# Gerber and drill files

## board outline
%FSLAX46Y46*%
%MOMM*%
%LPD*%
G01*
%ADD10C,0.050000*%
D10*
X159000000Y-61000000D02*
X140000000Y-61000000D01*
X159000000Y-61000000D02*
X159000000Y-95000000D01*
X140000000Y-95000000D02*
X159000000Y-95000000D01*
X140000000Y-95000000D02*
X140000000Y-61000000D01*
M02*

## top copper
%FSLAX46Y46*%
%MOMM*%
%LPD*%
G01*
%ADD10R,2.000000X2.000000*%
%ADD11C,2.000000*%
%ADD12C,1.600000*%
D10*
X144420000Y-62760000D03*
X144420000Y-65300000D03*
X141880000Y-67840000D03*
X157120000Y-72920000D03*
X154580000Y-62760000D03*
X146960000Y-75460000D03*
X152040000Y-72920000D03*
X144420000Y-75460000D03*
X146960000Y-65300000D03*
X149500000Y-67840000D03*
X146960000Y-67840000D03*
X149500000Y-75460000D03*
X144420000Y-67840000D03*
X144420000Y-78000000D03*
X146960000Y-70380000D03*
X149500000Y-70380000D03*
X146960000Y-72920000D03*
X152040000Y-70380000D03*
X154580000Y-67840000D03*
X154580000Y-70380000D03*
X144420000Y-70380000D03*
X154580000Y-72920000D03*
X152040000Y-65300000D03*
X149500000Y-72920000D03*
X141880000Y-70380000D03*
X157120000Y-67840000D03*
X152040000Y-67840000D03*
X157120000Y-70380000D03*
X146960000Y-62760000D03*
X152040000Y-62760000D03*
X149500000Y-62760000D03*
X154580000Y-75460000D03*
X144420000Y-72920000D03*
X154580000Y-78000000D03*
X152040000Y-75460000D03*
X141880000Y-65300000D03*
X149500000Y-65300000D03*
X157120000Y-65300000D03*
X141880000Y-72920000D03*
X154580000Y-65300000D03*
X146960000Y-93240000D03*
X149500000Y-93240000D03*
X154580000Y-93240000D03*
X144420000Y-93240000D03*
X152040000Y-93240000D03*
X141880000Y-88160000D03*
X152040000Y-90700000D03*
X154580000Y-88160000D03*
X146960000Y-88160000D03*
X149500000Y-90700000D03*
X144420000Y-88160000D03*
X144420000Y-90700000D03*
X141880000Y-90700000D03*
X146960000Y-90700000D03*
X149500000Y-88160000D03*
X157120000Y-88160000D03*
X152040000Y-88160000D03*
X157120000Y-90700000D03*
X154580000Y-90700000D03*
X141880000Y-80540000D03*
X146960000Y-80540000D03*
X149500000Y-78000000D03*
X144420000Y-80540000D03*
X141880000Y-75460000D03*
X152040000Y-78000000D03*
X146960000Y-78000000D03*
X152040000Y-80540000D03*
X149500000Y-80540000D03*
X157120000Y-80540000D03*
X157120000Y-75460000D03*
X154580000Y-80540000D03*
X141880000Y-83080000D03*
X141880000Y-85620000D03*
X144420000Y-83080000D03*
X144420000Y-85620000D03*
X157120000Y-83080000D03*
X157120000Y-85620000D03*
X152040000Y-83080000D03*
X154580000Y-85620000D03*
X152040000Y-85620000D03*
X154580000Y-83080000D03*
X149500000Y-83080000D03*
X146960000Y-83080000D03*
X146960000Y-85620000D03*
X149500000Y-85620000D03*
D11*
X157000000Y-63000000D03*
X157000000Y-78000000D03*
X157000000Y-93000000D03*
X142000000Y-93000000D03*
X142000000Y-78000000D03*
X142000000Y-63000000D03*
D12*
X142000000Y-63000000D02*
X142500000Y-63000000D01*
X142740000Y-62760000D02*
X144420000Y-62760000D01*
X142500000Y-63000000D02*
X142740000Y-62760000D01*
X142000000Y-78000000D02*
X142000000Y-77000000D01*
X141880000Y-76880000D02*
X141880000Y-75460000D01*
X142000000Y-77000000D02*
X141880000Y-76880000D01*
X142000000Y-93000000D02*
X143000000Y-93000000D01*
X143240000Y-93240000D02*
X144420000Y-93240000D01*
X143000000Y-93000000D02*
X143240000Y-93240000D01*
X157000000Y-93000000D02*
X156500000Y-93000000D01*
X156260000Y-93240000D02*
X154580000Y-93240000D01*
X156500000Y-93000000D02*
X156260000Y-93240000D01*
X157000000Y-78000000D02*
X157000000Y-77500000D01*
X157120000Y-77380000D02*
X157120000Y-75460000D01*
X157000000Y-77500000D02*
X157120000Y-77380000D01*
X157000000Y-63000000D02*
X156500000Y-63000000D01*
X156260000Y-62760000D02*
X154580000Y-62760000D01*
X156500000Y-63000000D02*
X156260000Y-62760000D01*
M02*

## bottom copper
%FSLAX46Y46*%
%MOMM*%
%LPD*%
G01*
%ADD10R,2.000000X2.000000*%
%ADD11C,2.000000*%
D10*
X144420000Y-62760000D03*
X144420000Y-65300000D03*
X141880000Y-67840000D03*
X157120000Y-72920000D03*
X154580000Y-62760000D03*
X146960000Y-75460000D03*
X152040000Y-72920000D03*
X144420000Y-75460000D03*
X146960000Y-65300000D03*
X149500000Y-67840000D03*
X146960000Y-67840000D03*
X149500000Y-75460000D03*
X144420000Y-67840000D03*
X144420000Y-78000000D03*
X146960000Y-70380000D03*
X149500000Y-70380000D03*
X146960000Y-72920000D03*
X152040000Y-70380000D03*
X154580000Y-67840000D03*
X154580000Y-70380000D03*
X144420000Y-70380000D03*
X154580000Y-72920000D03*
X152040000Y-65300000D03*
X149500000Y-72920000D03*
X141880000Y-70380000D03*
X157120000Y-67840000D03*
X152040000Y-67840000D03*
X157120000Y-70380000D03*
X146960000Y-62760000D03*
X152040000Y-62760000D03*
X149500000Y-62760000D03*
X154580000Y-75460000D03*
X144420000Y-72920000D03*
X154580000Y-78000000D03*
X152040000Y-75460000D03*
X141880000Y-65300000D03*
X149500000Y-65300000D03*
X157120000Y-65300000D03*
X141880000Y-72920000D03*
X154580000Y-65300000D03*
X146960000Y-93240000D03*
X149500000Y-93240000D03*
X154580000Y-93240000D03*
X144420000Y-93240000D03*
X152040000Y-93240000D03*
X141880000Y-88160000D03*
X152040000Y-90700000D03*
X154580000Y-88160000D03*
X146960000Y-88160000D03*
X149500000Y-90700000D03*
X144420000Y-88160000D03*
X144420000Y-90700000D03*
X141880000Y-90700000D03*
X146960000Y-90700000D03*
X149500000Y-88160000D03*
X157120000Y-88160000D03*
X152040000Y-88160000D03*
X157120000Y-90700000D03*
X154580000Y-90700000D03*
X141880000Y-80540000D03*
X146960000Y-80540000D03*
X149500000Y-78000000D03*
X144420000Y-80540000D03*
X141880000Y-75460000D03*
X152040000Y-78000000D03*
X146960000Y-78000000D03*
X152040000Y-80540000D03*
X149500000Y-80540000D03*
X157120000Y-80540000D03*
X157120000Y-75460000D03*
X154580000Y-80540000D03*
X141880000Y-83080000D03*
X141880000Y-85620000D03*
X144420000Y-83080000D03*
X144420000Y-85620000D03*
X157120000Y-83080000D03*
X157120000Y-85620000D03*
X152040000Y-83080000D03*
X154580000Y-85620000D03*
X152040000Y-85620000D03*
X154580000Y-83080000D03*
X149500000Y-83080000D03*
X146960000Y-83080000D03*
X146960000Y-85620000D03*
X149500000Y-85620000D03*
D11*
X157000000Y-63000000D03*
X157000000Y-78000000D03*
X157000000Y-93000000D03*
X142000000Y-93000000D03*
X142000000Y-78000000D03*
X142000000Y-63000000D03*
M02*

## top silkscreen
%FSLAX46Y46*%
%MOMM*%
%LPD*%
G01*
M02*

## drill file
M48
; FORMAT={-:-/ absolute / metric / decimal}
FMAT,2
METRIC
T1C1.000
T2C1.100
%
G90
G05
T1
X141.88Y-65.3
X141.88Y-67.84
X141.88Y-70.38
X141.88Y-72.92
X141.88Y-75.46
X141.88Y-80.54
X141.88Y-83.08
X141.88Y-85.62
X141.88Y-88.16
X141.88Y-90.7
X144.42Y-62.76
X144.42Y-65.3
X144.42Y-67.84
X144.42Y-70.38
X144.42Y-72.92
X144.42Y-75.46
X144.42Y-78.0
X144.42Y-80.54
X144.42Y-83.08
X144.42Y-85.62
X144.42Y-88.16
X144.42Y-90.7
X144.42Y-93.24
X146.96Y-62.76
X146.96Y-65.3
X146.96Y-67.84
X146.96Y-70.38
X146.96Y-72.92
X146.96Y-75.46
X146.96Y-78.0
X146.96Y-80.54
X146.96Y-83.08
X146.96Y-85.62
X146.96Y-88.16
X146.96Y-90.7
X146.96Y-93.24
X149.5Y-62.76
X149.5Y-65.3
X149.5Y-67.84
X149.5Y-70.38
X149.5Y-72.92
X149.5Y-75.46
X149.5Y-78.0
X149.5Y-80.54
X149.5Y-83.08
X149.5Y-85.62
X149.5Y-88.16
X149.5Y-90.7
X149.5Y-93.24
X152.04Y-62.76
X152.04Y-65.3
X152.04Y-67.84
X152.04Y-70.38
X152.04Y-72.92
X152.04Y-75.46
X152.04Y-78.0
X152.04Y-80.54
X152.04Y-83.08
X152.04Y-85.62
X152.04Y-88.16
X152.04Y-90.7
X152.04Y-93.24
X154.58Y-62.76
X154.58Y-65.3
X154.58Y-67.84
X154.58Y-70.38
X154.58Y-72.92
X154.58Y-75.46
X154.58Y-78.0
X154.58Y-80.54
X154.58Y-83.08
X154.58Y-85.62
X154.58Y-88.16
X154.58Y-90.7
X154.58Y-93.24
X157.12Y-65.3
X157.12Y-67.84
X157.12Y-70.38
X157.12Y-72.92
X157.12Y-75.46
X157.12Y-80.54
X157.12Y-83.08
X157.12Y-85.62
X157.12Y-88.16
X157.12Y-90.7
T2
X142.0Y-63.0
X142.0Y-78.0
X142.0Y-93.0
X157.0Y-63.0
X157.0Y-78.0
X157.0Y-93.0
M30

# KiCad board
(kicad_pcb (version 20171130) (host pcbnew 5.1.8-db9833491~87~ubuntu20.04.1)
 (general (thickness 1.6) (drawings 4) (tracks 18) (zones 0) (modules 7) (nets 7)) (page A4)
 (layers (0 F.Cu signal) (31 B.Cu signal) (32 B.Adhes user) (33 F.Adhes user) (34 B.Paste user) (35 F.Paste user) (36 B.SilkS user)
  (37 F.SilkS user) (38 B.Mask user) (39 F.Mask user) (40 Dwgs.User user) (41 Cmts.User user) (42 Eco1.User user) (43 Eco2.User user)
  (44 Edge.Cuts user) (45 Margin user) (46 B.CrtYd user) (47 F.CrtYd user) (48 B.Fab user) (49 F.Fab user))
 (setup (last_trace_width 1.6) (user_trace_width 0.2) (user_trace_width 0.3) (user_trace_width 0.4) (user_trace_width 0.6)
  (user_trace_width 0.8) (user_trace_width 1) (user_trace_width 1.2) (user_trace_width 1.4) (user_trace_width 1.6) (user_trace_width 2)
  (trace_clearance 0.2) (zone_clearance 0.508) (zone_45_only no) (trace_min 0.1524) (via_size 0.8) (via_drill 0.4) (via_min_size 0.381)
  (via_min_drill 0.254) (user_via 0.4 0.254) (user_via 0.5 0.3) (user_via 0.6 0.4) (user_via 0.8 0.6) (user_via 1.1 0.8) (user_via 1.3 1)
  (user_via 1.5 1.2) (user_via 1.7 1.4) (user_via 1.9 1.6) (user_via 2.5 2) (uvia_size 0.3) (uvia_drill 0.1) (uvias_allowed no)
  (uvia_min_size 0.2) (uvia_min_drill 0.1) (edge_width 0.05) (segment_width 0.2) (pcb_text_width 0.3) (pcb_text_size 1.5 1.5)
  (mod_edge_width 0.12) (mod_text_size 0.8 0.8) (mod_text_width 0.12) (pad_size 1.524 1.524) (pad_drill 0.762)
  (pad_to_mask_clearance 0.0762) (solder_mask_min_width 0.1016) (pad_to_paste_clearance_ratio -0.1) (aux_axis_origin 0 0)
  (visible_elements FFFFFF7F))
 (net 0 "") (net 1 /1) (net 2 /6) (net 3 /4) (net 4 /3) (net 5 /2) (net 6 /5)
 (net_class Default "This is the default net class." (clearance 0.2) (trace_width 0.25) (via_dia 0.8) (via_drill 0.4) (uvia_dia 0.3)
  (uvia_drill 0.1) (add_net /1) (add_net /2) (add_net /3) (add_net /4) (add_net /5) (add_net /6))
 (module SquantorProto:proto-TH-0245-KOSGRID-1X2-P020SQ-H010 (layer F.Cu) (at 149.5 78)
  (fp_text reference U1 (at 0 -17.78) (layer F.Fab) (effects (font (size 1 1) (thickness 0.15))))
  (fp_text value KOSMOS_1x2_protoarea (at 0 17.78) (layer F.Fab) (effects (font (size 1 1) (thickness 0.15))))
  (pad 1 thru_hole rect (at -5.08 -15.24) (size 2 2) (drill 1) (layers *.Cu *.Mask) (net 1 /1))
  (pad NC thru_hole rect (at -5.08 -12.7) (size 2 2) (drill 1) (layers *.Cu *.Mask))
  (pad NC thru_hole rect (at -7.62 -10.16) (size 2 2) (drill 1) (layers *.Cu *.Mask))
  (pad NC thru_hole rect (at 7.62 -5.08) (size 2 2) (drill 1) (layers *.Cu *.Mask))
  (pad 6 thru_hole rect (at 5.08 -15.24) (size 2 2) (drill 1) (layers *.Cu *.Mask) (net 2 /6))
  (pad NC thru_hole rect (at -2.54 -2.54) (size 2 2) (drill 1) (layers *.Cu *.Mask))
  (pad NC thru_hole rect (at 2.54 -5.08) (size 2 2) (drill 1) (layers *.Cu *.Mask))
  (pad NC thru_hole rect (at -5.08 -2.54) (size 2 2) (drill 1) (layers *.Cu *.Mask))
  (pad NC thru_hole rect (at -2.54 -12.7) (size 2 2) (drill 1) (layers *.Cu *.Mask))
  (pad NC thru_hole rect (at 0 -10.16) (size 2 2) (drill 1) (layers *.Cu *.Mask))
  (pad NC thru_hole rect (at -2.54 -10.16) (size 2 2) (drill 1) (layers *.Cu *.Mask))
  (pad NC thru_hole rect (at 0 -2.54) (size 2 2) (drill 1) (layers *.Cu *.Mask))
  (pad NC thru_hole rect (at -5.08 -10.16) (size 2 2) (drill 1) (layers *.Cu *.Mask))
  (pad NC thru_hole rect (at -5.08 0) (size 2 2) (drill 1) (layers *.Cu *.Mask))
  (pad NC thru_hole rect (at -2.54 -7.62) (size 2 2) (drill 1) (layers *.Cu *.Mask))
  (pad NC thru_hole rect (at 0 -7.62) (size 2 2) (drill 1) (layers *.Cu *.Mask))
  (pad NC thru_hole rect (at -2.54 -5.08) (size 2 2) (drill 1) (layers *.Cu *.Mask))
  (pad NC thru_hole rect (at 2.54 -7.62) (size 2 2) (drill 1) (layers *.Cu *.Mask))
  (pad NC thru_hole rect (at 5.08 -10.16) (size 2 2) (drill 1) (layers *.Cu *.Mask))
  (pad NC thru_hole rect (at 5.08 -7.62) (size 2 2) (drill 1) (layers *.Cu *.Mask))
  (pad NC thru_hole rect (at -5.08 -7.62) (size 2 2) (drill 1) (layers *.Cu *.Mask))
  (pad NC thru_hole rect (at 5.08 -5.08) (size 2 2) (drill 1) (layers *.Cu *.Mask))
  (pad NC thru_hole rect (at 2.54 -12.7) (size 2 2) (drill 1) (layers *.Cu *.Mask))
  (pad NC thru_hole rect (at 0 -5.08) (size 2 2) (drill 1) (layers *.Cu *.Mask))
  (pad NC thru_hole rect (at -7.62 -7.62) (size 2 2) (drill 1) (layers *.Cu *.Mask))
  (pad NC thru_hole rect (at 7.62 -10.16) (size 2 2) (drill 1) (layers *.Cu *.Mask))
  (pad NC thru_hole rect (at 2.54 -10.16) (size 2 2) (drill 1) (layers *.Cu *.Mask))
  (pad NC thru_hole rect (at 7.62 -7.62) (size 2 2) (drill 1) (layers *.Cu *.Mask))
  (pad NC thru_hole rect (at -2.54 -15.24) (size 2 2) (drill 1) (layers *.Cu *.Mask))
  (pad NC thru_hole rect (at 2.54 -15.24) (size 2 2) (drill 1) (layers *.Cu *.Mask))
  (pad NC thru_hole rect (at 0 -15.24) (size 2 2) (drill 1) (layers *.Cu *.Mask))
  (pad NC thru_hole rect (at 5.08 -2.54) (size 2 2) (drill 1) (layers *.Cu *.Mask))
  (pad NC thru_hole rect (at -5.08 -5.08) (size 2 2) (drill 1) (layers *.Cu *.Mask))
  (pad NC thru_hole rect (at 5.08 0) (size 2 2) (drill 1) (layers *.Cu *.Mask))
  (pad NC thru_hole rect (at 2.54 -2.54) (size 2 2) (drill 1) (layers *.Cu *.Mask))
  (pad NC thru_hole rect (at -7.62 -12.7) (size 2 2) (drill 1) (layers *.Cu *.Mask))
  (pad NC thru_hole rect (at 0 -12.7) (size 2 2) (drill 1) (layers *.Cu *.Mask))
  (pad NC thru_hole rect (at 7.62 -12.7) (size 2 2) (drill 1) (layers *.Cu *.Mask))
  (pad NC thru_hole rect (at -7.62 -5.08) (size 2 2) (drill 1) (layers *.Cu *.Mask))
  (pad NC thru_hole rect (at 5.08 -12.7) (size 2 2) (drill 1) (layers *.Cu *.Mask))
  (pad NC thru_hole rect (at -2.54 15.24) (size 2 2) (drill 1) (layers *.Cu *.Mask))
  (pad NC thru_hole rect (at 0 15.24) (size 2 2) (drill 1) (layers *.Cu *.Mask))
  (pad 4 thru_hole rect (at 5.08 15.24) (size 2 2) (drill 1) (layers *.Cu *.Mask) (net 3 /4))
  (pad 3 thru_hole rect (at -5.08 15.24) (size 2 2) (drill 1) (layers *.Cu *.Mask) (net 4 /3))
  (pad NC thru_hole rect (at 2.54 15.24) (size 2 2) (drill 1) (layers *.Cu *.Mask))
  (pad NC thru_hole rect (at -7.62 10.16) (size 2 2) (drill 1) (layers *.Cu *.Mask))
  (pad NC thru_hole rect (at 2.54 12.7) (size 2 2) (drill 1) (layers *.Cu *.Mask))
  (pad NC thru_hole rect (at 5.08 10.16) (size 2 2) (drill 1) (layers *.Cu *.Mask))
  (pad NC thru_hole rect (at -2.54 10.16) (size 2 2) (drill 1) (layers *.Cu *.Mask))
  (pad NC thru_hole rect (at 0 12.7) (size 2 2) (drill 1) (layers *.Cu *.Mask))
  (pad NC thru_hole rect (at -5.08 10.16) (size 2 2) (drill 1) (layers *.Cu *.Mask))
  (pad NC thru_hole rect (at -5.08 12.7) (size 2 2) (drill 1) (layers *.Cu *.Mask))
  (pad NC thru_hole rect (at -7.62 12.7) (size 2 2) (drill 1) (layers *.Cu *.Mask))
  (pad NC thru_hole rect (at -2.54 12.7) (size 2 2) (drill 1) (layers *.Cu *.Mask))
  (pad NC thru_hole rect (at 0 10.16) (size 2 2) (drill 1) (layers *.Cu *.Mask))
  (pad NC thru_hole rect (at 7.62 10.16) (size 2 2) (drill 1) (layers *.Cu *.Mask))
  (pad NC thru_hole rect (at 2.54 10.16) (size 2 2) (drill 1) (layers *.Cu *.Mask))
  (pad NC thru_hole rect (at 7.62 12.7) (size 2 2) (drill 1) (layers *.Cu *.Mask))
  (pad NC thru_hole rect (at 5.08 12.7) (size 2 2) (drill 1) (layers *.Cu *.Mask))
  (pad NC thru_hole rect (at -7.62 2.54) (size 2 2) (drill 1) (layers *.Cu *.Mask))
  (pad NC thru_hole rect (at -2.54 2.54) (size 2 2) (drill 1) (layers *.Cu *.Mask))
  (pad NC thru_hole rect (at 0 0) (size 2 2) (drill 1) (layers *.Cu *.Mask))
  (pad NC thru_hole rect (at -5.08 2.54) (size 2 2) (drill 1) (layers *.Cu *.Mask))
  (pad 2 thru_hole rect (at -7.62 -2.54) (size 2 2) (drill 1) (layers *.Cu *.Mask) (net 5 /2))
  (pad NC thru_hole rect (at 2.54 0) (size 2 2) (drill 1) (layers *.Cu *.Mask))
  (pad NC thru_hole rect (at -2.54 0) (size 2 2) (drill 1) (layers *.Cu *.Mask))
  (pad NC thru_hole rect (at 2.54 2.54) (size 2 2) (drill 1) (layers *.Cu *.Mask))
  (pad NC thru_hole rect (at 0 2.54) (size 2 2) (drill 1) (layers *.Cu *.Mask))
  (pad NC thru_hole rect (at 7.62 2.54) (size 2 2) (drill 1) (layers *.Cu *.Mask))
  (pad 5 thru_hole rect (at 7.62 -2.54) (size 2 2) (drill 1) (layers *.Cu *.Mask) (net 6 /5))
  (pad NC thru_hole rect (at 5.08 2.54) (size 2 2) (drill 1) (layers *.Cu *.Mask))
  (pad NC thru_hole rect (at -7.62 5.08) (size 2 2) (drill 1) (layers *.Cu *.Mask))
  (pad NC thru_hole rect (at -7.62 7.62) (size 2 2) (drill 1) (layers *.Cu *.Mask))
  (pad NC thru_hole rect (at -5.08 5.08) (size 2 2) (drill 1) (layers *.Cu *.Mask))
  (pad NC thru_hole rect (at -5.08 7.62) (size 2 2) (drill 1) (layers *.Cu *.Mask))
  (pad NC thru_hole rect (at 7.62 5.08) (size 2 2) (drill 1) (layers *.Cu *.Mask))
  (pad NC thru_hole rect (at 7.62 7.62) (size 2 2) (drill 1) (layers *.Cu *.Mask))
  (pad NC thru_hole rect (at 2.54 5.08) (size 2 2) (drill 1) (layers *.Cu *.Mask))
  (pad NC thru_hole rect (at 5.08 7.62) (size 2 2) (drill 1) (layers *.Cu *.Mask))
  (pad NC thru_hole rect (at 2.54 7.62) (size 2 2) (drill 1) (layers *.Cu *.Mask))
  (pad NC thru_hole rect (at 5.08 5.08) (size 2 2) (drill 1) (layers *.Cu *.Mask))
  (pad NC thru_hole rect (at 0 5.08) (size 2 2) (drill 1) (layers *.Cu *.Mask))
  (pad NC thru_hole rect (at -2.54 5.08) (size 2 2) (drill 1) (layers *.Cu *.Mask))
  (pad NC thru_hole rect (at -2.54 7.62) (size 2 2) (drill 1) (layers *.Cu *.Mask))
  (pad NC thru_hole rect (at 0 7.62) (size 2 2) (drill 1) (layers *.Cu *.Mask)))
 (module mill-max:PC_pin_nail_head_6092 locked (layer F.Cu) (at 157 63)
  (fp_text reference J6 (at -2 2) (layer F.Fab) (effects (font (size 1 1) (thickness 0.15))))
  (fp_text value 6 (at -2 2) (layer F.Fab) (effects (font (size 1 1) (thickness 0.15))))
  (pad 1 thru_hole circle (at 0 0) (size 2 2) (drill 1.1) (layers *.Cu *.Mask) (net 2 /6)))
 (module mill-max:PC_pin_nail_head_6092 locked (layer F.Cu) (at 157 78)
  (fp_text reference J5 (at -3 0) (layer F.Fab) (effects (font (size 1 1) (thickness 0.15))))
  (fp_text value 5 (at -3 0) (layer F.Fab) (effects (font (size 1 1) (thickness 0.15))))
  (pad 1 thru_hole circle (at 0 0) (size 2 2) (drill 1.1) (layers *.Cu *.Mask) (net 6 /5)))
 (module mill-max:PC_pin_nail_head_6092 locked (layer F.Cu) (at 157 93)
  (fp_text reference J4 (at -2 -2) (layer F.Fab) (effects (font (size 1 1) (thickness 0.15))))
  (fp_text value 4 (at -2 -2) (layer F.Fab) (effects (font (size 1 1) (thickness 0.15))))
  (pad 1 thru_hole circle (at 0 0) (size 2 2) (drill 1.1) (layers *.Cu *.Mask) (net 3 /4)))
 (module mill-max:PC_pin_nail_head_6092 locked (layer F.Cu) (at 142 93)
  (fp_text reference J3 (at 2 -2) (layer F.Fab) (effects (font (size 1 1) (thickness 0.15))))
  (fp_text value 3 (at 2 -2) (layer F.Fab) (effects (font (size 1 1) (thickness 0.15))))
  (pad 1 thru_hole circle (at 0 0) (size 2 2) (drill 1.1) (layers *.Cu *.Mask) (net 4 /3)))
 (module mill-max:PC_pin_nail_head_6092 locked (layer F.Cu) (at 142 78)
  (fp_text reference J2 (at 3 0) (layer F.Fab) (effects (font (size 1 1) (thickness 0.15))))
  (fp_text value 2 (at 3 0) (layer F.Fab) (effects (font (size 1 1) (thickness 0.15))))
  (pad 1 thru_hole circle (at 0 0) (size 2 2) (drill 1.1) (layers *.Cu *.Mask) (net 5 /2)))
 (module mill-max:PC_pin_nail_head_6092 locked (layer F.Cu) (at 142 63)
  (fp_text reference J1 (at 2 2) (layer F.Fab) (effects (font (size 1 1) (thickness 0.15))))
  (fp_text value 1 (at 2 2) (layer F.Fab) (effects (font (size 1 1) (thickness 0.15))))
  (pad 1 thru_hole circle (at 0 0) (size 2 2) (drill 1.1) (layers *.Cu *.Mask) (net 1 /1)))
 (gr_line (start 159 61) (end 140 61) (layer Edge.Cuts) (width 0.05))
 (gr_line (start 159 61) (end 159 95) (layer Edge.Cuts) (width 0.05))
 (gr_line (start 140 95) (end 159 95) (layer Edge.Cuts) (width 0.05))
 (gr_line (start 140 95) (end 140 61) (layer Edge.Cuts) (width 0.05))
 (segment (start 142 63) (end 142.5 63) (width 1.6) (layer F.Cu) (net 1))
 (segment (start 142.74 62.76) (end 144.42 62.76) (width 1.6) (layer F.Cu) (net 1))
 (segment (start 142.5 63) (end 142.74 62.76) (width 1.6) (layer F.Cu) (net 1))
 (segment (start 142 78) (end 142 77) (width 1.6) (layer F.Cu) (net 5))
 (segment (start 141.88 76.88) (end 141.88 75.46) (width 1.6) (layer F.Cu) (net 5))
 (segment (start 142 77) (end 141.88 76.88) (width 1.6) (layer F.Cu) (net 5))
 (segment (start 142 93) (end 143 93) (width 1.6) (layer F.Cu) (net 4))
 (segment (start 143.24 93.24) (end 144.42 93.24) (width 1.6) (layer F.Cu) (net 4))
 (segment (start 143 93) (end 143.24 93.24) (width 1.6) (layer F.Cu) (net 4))
 (segment (start 157 93) (end 156.5 93) (width 1.6) (layer F.Cu) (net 3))
 (segment (start 156.26 93.24) (end 154.58 93.24) (width 1.6) (layer F.Cu) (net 3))
 (segment (start 156.5 93) (end 156.26 93.24) (width 1.6) (layer F.Cu) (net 3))
 (segment (start 157 78) (end 157 77.5) (width 1.6) (layer F.Cu) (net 6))
 (segment (start 157.12 77.38) (end 157.12 75.46) (width 1.6) (layer F.Cu) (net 6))
 (segment (start 157 77.5) (end 157.12 77.38) (width 1.6) (layer F.Cu) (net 6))
 (segment (start 157 63) (end 156.5 63) (width 1.6) (layer F.Cu) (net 2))
 (segment (start 156.26 62.76) (end 154.58 62.76) (width 1.6) (layer F.Cu) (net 2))
 (segment (start 156.5 63) (end 156.26 62.76) (width 1.6) (layer F.Cu) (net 2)))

